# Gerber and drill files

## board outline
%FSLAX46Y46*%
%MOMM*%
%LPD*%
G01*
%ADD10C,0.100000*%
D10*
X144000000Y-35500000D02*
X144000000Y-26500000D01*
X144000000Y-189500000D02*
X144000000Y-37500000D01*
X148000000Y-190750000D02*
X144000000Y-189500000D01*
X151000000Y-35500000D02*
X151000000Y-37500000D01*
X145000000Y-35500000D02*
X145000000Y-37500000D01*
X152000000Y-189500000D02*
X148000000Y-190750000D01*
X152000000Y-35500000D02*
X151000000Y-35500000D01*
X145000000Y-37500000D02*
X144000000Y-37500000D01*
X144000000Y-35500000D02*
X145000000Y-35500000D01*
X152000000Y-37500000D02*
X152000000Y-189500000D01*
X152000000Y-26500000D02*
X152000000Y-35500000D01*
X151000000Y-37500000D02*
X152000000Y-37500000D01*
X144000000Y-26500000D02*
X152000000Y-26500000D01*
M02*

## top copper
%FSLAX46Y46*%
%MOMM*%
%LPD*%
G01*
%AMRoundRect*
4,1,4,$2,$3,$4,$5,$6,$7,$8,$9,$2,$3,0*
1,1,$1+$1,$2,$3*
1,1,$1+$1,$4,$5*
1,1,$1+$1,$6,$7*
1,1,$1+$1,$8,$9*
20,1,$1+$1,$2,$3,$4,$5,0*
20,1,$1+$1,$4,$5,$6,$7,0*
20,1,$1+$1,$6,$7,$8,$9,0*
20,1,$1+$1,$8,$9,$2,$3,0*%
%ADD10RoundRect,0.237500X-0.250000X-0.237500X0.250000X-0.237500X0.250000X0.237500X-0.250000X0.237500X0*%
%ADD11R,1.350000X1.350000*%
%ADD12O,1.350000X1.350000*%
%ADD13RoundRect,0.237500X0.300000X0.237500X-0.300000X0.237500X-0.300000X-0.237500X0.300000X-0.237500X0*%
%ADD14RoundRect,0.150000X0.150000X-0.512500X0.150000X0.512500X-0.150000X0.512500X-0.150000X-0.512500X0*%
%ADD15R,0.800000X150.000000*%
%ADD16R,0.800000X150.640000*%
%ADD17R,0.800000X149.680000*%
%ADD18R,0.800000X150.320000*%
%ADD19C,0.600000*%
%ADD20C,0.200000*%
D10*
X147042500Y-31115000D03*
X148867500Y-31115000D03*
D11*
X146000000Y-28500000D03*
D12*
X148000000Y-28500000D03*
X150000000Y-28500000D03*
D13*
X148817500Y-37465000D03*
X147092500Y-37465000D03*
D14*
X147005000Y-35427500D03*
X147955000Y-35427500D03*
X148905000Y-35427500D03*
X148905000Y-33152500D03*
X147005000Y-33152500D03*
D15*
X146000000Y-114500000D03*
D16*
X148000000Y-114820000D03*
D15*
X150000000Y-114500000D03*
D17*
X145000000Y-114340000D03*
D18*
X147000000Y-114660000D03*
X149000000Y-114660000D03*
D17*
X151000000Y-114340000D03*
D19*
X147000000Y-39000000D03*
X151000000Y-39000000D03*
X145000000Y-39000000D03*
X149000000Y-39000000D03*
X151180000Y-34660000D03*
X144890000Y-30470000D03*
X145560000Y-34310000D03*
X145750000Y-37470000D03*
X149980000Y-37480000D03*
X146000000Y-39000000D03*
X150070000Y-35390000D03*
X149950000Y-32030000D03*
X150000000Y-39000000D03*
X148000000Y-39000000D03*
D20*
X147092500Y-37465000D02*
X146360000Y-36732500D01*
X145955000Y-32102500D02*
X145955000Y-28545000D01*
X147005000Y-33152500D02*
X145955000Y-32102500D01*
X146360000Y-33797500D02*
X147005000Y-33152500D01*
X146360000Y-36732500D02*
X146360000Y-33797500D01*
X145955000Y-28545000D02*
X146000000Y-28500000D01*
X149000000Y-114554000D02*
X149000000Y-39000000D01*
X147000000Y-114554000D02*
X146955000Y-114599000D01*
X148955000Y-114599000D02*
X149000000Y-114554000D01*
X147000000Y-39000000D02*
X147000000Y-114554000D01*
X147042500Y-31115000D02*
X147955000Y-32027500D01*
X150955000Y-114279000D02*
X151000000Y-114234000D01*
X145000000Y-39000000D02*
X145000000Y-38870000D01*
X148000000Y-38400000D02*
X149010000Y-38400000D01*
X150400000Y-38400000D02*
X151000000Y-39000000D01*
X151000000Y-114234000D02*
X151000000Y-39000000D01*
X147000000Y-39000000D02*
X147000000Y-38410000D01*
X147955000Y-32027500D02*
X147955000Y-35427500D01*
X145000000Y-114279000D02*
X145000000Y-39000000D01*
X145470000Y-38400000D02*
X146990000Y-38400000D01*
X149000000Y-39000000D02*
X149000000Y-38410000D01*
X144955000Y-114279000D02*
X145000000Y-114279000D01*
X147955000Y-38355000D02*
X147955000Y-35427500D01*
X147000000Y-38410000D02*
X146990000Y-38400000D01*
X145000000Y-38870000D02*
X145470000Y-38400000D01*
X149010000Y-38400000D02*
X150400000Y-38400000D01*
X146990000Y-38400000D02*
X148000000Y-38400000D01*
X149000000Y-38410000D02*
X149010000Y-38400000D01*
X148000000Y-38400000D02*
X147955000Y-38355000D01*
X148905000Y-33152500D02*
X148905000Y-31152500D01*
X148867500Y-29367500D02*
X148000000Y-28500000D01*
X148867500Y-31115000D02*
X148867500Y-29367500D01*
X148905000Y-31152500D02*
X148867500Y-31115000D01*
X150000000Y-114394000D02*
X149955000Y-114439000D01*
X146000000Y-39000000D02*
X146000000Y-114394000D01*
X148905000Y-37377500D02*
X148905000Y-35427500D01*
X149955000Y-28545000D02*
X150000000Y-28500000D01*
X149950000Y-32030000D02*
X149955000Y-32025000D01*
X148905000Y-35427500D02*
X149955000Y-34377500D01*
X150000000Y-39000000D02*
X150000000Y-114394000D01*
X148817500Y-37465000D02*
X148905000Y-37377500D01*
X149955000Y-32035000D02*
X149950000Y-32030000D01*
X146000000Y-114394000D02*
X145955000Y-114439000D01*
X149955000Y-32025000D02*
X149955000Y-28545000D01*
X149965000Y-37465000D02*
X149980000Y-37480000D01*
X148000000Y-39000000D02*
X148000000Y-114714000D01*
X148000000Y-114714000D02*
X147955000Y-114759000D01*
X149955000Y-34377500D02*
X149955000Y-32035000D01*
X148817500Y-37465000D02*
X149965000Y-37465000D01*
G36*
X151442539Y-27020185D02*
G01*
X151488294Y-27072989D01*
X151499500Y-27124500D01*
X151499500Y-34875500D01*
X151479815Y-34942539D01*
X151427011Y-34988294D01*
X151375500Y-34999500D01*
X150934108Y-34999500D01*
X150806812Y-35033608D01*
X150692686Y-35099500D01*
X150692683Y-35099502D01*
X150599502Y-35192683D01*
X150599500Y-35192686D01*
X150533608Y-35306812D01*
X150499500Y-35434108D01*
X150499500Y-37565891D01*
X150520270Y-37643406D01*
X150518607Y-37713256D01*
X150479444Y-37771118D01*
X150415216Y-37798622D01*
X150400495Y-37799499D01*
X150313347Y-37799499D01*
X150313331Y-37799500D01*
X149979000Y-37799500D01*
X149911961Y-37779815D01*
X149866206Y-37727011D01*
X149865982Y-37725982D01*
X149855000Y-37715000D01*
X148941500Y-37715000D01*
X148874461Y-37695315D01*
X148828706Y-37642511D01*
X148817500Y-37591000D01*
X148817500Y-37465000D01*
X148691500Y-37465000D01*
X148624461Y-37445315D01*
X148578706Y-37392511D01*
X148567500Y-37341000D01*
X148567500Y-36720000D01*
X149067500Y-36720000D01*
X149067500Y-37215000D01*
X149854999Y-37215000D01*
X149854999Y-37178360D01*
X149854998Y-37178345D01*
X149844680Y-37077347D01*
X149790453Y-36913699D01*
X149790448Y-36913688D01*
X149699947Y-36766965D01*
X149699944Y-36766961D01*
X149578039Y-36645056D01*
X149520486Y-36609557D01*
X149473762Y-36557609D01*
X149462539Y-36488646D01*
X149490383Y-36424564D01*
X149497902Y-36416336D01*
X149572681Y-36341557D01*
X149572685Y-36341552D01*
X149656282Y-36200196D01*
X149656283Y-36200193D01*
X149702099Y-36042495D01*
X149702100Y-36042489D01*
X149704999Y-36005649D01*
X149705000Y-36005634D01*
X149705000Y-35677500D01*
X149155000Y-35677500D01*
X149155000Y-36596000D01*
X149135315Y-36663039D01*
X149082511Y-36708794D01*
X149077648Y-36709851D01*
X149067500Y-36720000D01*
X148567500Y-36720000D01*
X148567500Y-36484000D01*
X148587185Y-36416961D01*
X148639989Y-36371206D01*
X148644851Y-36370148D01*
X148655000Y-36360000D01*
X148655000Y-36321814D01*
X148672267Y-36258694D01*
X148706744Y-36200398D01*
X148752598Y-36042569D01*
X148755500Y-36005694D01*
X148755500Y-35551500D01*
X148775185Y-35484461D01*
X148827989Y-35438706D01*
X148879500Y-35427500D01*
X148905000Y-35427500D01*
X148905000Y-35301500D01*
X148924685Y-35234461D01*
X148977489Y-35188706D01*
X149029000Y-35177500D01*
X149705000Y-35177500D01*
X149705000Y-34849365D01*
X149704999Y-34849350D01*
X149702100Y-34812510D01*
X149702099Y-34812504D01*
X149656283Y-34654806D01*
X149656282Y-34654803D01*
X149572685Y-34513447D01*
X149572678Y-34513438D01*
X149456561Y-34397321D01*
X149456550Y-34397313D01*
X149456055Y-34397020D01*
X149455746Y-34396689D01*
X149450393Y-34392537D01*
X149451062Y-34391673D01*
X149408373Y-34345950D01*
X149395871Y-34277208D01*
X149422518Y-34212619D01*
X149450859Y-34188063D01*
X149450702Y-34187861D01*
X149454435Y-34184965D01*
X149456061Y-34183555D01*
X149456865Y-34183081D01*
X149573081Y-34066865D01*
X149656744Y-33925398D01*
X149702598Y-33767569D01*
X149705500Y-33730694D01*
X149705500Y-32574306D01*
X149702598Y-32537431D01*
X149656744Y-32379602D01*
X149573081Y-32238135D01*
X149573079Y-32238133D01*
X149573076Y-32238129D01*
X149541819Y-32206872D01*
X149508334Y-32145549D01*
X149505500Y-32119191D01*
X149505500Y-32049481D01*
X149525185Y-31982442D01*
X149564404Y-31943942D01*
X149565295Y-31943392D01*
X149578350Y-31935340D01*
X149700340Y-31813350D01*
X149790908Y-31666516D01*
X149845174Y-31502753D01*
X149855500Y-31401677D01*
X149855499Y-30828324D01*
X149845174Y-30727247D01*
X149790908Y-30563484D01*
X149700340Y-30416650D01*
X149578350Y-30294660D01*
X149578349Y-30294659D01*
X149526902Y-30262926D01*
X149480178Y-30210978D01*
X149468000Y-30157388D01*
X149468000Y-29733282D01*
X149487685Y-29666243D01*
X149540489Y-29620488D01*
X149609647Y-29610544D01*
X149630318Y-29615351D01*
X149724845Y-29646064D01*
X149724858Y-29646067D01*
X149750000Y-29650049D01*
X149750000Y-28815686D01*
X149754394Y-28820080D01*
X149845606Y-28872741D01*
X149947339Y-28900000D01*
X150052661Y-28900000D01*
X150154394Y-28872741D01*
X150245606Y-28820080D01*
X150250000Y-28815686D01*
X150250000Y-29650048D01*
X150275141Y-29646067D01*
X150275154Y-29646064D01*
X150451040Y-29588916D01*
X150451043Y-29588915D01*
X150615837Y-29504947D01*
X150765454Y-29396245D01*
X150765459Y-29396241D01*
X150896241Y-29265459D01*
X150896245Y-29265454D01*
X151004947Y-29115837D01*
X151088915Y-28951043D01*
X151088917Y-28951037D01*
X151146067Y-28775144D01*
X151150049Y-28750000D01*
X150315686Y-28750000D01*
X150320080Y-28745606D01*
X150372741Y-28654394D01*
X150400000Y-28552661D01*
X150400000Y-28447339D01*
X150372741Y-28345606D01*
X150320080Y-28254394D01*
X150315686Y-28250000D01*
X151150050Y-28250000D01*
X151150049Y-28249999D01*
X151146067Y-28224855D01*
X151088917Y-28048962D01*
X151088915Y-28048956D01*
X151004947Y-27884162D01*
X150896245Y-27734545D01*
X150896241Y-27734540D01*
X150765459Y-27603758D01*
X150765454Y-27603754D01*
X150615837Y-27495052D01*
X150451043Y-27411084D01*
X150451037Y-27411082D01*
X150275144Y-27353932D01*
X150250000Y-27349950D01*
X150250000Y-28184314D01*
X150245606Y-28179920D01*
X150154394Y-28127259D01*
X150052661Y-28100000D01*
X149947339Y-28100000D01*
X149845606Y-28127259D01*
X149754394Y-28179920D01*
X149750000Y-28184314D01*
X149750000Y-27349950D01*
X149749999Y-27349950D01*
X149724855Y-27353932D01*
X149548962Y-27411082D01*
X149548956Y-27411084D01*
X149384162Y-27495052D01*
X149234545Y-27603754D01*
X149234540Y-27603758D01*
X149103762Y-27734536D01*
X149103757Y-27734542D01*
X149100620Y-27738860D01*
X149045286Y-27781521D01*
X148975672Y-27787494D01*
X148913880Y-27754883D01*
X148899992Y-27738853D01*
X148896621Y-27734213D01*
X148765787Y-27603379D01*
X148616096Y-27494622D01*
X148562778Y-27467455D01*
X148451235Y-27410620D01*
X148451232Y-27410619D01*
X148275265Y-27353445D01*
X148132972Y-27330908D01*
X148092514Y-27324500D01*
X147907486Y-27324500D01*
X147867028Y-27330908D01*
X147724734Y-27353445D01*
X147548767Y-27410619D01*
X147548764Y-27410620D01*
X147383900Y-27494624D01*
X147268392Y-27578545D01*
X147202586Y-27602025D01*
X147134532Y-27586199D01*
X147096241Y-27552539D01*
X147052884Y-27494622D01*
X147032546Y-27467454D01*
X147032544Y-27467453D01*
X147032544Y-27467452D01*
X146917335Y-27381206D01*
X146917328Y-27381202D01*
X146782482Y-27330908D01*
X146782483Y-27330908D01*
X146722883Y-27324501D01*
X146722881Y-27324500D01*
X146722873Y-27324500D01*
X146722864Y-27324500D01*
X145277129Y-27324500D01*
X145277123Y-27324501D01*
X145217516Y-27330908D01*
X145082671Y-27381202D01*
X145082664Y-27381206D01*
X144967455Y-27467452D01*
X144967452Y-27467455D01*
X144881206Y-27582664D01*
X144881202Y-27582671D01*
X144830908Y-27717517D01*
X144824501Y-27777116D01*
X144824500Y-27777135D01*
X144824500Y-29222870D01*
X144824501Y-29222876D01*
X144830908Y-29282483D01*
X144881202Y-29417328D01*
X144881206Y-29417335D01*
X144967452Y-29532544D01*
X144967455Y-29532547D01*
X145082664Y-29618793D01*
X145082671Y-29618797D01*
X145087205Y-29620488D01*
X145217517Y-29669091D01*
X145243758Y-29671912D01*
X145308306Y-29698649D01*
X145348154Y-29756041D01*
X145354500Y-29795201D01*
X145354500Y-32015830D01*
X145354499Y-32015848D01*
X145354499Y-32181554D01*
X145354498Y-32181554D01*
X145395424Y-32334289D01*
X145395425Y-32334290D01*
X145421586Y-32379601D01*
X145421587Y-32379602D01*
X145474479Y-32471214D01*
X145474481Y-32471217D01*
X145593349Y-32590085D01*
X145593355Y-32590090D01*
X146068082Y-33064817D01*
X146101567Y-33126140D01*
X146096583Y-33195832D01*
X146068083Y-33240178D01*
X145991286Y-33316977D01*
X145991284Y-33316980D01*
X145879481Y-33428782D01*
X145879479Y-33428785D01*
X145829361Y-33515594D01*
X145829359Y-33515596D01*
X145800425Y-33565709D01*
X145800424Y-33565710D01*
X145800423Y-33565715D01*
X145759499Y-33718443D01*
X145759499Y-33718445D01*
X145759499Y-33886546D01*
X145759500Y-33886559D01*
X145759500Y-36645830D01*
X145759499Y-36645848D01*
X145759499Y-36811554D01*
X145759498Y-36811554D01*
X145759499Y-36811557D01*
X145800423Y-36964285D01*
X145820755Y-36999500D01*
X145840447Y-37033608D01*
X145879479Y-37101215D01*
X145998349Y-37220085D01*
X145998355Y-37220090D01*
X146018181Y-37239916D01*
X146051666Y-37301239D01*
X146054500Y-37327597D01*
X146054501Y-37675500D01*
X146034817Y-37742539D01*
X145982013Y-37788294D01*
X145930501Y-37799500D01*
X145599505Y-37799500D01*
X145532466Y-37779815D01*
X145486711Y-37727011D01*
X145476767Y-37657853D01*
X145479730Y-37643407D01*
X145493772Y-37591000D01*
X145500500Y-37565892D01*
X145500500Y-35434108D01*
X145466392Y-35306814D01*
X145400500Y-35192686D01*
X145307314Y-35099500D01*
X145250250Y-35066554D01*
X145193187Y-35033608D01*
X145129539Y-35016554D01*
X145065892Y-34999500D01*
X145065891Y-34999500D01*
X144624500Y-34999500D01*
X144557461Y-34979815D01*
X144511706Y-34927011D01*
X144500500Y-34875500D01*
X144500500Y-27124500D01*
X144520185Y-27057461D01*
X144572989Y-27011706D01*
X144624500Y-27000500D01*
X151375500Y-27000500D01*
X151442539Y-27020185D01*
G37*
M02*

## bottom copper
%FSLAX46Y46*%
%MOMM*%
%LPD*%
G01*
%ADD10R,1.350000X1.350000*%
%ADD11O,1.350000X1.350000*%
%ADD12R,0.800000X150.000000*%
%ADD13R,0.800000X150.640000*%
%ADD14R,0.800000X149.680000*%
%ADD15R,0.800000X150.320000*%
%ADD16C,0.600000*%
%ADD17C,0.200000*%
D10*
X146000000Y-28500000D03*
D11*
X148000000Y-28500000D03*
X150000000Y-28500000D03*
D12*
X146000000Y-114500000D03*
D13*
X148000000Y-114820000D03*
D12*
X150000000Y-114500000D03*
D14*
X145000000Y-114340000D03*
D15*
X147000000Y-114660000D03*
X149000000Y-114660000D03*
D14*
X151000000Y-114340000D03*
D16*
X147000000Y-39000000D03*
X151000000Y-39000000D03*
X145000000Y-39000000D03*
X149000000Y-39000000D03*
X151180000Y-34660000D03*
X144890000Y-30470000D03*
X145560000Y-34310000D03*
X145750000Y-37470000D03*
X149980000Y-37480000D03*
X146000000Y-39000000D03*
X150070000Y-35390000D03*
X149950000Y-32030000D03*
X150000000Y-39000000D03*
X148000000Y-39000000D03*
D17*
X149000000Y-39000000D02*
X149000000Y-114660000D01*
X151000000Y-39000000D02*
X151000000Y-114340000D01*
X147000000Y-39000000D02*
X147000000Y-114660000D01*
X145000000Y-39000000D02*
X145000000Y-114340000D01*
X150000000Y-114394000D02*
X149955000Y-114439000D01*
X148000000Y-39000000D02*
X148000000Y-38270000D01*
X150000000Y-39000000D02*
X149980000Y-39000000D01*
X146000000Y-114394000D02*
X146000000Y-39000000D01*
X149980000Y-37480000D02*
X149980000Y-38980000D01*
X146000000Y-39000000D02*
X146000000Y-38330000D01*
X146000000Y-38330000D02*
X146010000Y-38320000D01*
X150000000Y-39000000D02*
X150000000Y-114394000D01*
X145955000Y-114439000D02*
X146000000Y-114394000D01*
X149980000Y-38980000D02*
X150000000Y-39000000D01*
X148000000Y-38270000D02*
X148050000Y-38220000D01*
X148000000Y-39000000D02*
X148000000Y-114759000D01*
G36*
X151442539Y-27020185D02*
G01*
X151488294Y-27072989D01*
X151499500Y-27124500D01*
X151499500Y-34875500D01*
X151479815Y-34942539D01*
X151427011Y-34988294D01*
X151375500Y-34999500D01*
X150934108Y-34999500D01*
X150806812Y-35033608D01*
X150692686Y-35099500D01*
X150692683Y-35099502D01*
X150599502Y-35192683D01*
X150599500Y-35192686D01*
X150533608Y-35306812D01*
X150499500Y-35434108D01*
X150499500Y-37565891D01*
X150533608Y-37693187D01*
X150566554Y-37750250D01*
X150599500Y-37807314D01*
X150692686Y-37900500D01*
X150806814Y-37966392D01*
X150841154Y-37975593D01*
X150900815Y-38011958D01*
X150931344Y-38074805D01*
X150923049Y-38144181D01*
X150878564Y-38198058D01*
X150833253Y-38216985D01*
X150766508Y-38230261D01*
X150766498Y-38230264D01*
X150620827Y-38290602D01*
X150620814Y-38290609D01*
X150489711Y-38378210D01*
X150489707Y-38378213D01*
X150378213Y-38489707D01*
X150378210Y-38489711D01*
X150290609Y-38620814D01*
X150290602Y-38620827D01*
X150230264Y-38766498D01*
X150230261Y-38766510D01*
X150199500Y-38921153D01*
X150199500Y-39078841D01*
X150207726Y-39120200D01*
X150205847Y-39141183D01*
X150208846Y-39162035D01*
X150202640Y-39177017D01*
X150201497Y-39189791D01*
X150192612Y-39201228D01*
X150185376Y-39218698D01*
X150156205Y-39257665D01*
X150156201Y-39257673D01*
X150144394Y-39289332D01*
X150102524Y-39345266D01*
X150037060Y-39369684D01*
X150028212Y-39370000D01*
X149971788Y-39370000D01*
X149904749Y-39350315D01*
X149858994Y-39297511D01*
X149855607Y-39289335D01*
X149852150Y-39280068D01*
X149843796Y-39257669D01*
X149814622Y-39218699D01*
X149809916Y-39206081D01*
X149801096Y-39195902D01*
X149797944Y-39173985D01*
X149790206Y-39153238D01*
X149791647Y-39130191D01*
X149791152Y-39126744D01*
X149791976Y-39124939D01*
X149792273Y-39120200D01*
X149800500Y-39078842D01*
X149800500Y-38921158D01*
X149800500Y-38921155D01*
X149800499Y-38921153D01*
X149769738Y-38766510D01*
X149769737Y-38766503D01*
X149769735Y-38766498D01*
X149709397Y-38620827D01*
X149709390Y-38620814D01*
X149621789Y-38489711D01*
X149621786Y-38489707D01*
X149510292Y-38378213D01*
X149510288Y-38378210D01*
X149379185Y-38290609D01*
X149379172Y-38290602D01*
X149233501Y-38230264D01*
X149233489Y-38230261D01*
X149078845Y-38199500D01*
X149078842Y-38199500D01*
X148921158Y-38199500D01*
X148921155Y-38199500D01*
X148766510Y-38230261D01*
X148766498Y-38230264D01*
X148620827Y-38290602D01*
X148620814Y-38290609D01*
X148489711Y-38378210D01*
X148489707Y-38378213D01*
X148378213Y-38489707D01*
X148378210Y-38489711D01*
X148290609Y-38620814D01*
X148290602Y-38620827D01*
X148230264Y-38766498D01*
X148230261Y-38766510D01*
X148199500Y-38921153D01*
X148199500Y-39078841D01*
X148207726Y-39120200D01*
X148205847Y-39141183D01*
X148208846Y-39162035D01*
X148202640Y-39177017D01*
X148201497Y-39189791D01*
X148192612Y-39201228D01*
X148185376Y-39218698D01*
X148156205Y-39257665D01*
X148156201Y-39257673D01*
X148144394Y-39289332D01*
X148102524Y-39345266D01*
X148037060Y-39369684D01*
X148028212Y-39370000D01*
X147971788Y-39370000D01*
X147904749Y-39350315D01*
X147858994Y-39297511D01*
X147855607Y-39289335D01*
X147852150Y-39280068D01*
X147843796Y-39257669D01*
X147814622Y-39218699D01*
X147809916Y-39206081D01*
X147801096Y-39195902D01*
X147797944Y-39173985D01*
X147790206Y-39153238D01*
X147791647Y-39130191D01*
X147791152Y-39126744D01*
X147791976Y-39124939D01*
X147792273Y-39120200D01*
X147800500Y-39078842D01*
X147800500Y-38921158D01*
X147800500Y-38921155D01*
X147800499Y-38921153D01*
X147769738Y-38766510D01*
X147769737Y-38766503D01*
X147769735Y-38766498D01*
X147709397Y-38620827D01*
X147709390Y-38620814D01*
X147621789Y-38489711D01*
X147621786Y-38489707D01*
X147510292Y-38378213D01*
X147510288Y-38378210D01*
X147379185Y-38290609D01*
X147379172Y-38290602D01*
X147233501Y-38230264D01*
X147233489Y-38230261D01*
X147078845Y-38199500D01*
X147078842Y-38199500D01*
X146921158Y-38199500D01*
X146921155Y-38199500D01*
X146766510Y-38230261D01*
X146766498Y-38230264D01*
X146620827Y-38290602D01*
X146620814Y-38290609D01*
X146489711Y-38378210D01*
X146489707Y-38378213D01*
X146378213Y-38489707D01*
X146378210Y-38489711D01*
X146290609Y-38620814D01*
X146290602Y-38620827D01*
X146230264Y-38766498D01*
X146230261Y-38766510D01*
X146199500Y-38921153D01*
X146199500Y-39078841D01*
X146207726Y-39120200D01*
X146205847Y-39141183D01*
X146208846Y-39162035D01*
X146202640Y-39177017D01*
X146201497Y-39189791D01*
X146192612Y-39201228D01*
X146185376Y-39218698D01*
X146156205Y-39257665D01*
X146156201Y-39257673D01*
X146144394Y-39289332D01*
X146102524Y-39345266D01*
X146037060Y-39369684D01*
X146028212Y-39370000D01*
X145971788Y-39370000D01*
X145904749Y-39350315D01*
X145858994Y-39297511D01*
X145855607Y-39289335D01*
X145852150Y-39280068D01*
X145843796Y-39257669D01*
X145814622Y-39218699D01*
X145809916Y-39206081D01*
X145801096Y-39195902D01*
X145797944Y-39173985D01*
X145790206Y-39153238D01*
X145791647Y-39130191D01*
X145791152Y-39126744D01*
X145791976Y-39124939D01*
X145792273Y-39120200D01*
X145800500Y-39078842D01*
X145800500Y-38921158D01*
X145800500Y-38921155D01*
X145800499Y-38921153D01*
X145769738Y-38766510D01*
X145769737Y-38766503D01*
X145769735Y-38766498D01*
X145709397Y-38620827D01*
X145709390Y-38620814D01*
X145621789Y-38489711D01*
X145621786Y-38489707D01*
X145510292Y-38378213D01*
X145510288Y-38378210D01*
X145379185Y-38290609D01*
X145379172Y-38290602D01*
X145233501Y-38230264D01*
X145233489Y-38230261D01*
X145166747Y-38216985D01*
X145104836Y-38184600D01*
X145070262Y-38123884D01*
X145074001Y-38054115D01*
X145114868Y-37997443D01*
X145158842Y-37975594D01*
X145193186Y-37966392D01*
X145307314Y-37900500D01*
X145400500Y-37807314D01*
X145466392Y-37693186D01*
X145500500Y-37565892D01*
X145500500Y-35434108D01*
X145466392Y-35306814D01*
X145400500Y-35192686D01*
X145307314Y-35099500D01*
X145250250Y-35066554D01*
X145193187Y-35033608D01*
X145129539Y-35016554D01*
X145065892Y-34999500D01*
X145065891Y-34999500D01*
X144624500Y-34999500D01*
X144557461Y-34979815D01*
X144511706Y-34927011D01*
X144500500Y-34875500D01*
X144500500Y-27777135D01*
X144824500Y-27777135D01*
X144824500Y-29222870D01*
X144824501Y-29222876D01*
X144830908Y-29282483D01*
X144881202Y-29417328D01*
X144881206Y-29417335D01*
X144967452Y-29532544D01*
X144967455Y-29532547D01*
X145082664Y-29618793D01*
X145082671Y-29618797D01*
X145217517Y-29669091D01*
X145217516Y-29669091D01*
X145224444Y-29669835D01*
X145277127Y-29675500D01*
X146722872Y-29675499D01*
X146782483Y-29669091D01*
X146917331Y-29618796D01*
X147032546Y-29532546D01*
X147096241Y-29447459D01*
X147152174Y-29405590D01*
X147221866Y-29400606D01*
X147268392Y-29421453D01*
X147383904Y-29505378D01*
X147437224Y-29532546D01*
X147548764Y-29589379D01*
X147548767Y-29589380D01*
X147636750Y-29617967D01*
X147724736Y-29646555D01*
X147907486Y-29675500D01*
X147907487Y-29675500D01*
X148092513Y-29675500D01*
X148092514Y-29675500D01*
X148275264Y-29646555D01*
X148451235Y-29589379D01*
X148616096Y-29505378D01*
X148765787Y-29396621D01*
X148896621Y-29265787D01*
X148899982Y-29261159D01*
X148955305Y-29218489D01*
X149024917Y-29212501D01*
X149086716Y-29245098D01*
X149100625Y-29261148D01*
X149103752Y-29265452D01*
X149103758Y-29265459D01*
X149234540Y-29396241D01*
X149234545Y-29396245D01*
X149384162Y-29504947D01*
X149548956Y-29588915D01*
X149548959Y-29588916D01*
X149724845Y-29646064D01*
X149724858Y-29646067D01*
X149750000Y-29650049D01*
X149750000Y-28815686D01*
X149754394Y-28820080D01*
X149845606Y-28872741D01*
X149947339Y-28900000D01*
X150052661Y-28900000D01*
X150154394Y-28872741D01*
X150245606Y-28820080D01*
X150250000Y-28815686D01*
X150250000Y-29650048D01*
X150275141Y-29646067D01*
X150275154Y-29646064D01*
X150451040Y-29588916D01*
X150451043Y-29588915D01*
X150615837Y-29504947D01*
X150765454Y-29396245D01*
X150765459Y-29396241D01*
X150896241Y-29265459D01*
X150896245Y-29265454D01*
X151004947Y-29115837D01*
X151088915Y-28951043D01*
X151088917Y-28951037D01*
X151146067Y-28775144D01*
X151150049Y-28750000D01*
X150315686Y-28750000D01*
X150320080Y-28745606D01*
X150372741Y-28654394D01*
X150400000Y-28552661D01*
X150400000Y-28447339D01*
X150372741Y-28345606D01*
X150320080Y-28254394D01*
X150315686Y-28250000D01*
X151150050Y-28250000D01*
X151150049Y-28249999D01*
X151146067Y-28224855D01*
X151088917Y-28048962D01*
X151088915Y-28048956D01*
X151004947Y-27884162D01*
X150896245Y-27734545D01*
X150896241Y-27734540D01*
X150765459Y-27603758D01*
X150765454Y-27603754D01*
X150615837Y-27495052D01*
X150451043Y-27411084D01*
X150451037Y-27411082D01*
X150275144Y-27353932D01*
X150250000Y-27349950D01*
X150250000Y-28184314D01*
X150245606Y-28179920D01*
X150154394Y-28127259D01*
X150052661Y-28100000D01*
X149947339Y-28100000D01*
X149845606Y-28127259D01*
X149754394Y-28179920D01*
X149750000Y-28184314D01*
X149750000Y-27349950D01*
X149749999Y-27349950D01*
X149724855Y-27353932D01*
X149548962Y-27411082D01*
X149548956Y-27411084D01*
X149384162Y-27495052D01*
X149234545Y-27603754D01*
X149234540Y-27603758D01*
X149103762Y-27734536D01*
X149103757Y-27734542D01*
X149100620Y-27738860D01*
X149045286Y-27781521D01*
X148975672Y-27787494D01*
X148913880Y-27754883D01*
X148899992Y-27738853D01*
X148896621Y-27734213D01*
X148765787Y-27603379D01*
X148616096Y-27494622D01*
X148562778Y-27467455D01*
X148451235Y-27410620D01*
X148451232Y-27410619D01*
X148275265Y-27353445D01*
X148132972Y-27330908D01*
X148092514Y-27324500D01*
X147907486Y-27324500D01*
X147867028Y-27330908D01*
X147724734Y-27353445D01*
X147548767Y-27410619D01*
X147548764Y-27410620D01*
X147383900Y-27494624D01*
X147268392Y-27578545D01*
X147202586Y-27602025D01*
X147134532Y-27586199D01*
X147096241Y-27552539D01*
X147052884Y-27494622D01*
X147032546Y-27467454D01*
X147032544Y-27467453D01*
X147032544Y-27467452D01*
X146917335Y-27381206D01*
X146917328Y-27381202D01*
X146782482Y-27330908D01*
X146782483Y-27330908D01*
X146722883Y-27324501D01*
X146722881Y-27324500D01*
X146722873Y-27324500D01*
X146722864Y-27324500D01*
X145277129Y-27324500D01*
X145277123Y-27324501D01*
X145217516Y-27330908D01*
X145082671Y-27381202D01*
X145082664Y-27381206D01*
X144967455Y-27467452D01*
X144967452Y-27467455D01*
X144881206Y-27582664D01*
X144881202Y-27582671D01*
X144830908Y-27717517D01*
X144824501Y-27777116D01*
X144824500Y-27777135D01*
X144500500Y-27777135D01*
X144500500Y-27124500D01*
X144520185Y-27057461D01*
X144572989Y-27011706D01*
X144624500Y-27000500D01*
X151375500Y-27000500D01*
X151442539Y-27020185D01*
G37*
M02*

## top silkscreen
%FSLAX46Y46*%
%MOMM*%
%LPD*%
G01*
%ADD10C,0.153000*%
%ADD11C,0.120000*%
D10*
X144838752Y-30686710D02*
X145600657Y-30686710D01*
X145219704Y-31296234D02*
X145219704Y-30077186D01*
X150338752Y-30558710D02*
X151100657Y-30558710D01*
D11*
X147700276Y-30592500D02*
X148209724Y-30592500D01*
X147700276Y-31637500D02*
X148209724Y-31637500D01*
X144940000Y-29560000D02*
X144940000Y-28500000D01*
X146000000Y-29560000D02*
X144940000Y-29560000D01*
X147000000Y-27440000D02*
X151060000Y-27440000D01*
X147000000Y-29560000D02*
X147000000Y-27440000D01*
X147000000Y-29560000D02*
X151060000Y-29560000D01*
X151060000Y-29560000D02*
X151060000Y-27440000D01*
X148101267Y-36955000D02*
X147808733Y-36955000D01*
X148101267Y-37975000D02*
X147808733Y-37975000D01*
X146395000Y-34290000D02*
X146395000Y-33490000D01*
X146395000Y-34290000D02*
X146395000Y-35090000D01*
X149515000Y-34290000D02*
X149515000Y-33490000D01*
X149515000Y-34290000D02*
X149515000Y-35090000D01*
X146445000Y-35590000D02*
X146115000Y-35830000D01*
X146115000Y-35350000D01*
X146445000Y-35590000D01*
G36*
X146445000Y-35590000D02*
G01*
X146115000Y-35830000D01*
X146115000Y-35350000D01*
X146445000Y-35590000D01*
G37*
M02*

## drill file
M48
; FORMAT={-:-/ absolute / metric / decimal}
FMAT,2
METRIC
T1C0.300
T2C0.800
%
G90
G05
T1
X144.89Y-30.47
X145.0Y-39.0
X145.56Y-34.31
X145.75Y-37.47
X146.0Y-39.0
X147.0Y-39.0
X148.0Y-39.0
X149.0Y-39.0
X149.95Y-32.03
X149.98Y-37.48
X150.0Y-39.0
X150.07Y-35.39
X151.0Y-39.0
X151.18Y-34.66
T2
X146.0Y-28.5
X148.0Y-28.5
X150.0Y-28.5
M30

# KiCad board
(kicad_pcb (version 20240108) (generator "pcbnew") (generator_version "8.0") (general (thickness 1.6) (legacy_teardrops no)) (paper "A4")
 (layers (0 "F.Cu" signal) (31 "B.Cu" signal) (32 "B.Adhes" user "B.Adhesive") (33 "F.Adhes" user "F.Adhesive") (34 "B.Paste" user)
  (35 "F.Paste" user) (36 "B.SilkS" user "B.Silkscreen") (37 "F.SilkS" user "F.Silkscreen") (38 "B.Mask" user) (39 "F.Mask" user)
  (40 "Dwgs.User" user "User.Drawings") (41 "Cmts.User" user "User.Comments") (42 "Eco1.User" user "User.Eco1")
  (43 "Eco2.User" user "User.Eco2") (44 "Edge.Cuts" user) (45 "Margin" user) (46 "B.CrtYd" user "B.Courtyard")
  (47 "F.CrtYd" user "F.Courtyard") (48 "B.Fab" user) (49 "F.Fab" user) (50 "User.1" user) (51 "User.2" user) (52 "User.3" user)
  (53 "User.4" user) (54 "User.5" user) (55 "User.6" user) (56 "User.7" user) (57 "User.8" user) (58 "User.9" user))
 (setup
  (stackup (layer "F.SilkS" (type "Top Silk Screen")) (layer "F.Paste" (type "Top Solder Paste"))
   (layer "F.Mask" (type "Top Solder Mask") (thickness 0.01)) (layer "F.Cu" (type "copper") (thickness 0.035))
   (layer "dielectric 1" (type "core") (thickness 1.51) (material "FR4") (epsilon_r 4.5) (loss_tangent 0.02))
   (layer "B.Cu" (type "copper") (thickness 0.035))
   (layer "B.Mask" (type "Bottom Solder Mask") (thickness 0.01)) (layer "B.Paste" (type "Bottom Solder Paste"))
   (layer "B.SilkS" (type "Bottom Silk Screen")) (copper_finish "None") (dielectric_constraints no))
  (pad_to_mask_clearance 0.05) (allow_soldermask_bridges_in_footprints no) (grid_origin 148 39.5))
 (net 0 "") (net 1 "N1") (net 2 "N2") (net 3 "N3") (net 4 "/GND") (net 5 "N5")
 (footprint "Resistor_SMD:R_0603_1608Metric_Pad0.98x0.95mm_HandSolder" (layer "F.Cu") (at 147.955 31.115)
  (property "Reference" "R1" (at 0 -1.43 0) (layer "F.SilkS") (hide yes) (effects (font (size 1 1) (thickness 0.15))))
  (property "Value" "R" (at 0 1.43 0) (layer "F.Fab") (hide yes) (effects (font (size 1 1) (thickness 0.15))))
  (fp_line (start -0.254724 -0.5225) (end 0.254724 -0.5225) (stroke (width 0.12) (type solid)) (layer "F.SilkS"))
  (fp_line (start -0.254724 0.5225) (end 0.254724 0.5225) (stroke (width 0.12) (type solid)) (layer "F.SilkS"))
  (pad "1" smd roundrect (at -0.9125 0) (size 0.975 0.95) (layers "F.Cu" "F.Paste" "F.Mask") (roundrect_rratio 0.25) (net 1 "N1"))
  (pad "2" smd roundrect (at 0.9125 0) (size 0.975 0.95) (layers "F.Cu" "F.Paste" "F.Mask") (roundrect_rratio 0.25) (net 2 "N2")))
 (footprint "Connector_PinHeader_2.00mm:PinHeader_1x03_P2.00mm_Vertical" (layer "F.Cu") (at 146 28.5 90)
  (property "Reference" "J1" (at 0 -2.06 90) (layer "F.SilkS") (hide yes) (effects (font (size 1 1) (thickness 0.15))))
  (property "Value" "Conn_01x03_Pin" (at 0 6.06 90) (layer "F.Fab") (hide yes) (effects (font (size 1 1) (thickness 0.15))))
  (fp_line (start -1.06 -1.06) (end 0 -1.06) (stroke (width 0.12) (type solid)) (layer "F.SilkS"))
  (fp_line (start -1.06 0) (end -1.06 -1.06) (stroke (width 0.12) (type solid)) (layer "F.SilkS"))
  (fp_line (start 1.06 1) (end 1.06 5.06) (stroke (width 0.12) (type solid)) (layer "F.SilkS"))
  (fp_line (start -1.06 1) (end 1.06 1) (stroke (width 0.12) (type solid)) (layer "F.SilkS"))
  (fp_line (start -1.06 1) (end -1.06 5.06) (stroke (width 0.12) (type solid)) (layer "F.SilkS"))
  (fp_line (start -1.06 5.06) (end 1.06 5.06) (stroke (width 0.12) (type solid)) (layer "F.SilkS"))
  (pad "1" thru_hole rect (at 0 0 90) (size 1.35 1.35) (drill 0.8) (layers "*.Cu" "*.Mask") (remove_unused_layers no) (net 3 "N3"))
  (pad "2" thru_hole oval (at 0 2 90) (size 1.35 1.35) (drill 0.8) (layers "*.Cu" "*.Mask") (remove_unused_layers no) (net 2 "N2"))
  (pad "3" thru_hole oval (at 0 4 90) (size 1.35 1.35) (drill 0.8) (layers "*.Cu" "*.Mask") (remove_unused_layers no) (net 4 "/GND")))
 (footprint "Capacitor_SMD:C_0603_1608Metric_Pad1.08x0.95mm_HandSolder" (layer "F.Cu") (at 147.955 37.465 180)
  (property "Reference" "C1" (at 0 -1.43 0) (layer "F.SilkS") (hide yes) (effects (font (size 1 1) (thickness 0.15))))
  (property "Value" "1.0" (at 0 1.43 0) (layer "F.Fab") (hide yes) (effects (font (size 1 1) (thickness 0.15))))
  (fp_line (start -0.146267 0.51) (end 0.146267 0.51) (stroke (width 0.12) (type solid)) (layer "F.SilkS"))
  (fp_line (start -0.146267 -0.51) (end 0.146267 -0.51) (stroke (width 0.12) (type solid)) (layer "F.SilkS"))
  (pad "1" smd roundrect (at -0.8625 0 180) (size 1.075 0.95) (layers "F.Cu" "F.Paste" "F.Mask") (roundrect_rratio 0.25) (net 4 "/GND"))
  (pad "2" smd roundrect (at 0.8625 0 180) (size 1.075 0.95) (layers "F.Cu" "F.Paste" "F.Mask") (roundrect_rratio 0.25) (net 3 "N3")))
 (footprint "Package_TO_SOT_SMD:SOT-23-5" (layer "F.Cu") (at 147.955 34.29 90)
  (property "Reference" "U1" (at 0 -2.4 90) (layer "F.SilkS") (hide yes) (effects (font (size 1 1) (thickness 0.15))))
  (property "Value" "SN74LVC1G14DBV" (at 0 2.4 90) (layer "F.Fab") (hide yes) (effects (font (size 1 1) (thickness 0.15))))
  (fp_line (start 0 -1.56) (end 0.8 -1.56) (stroke (width 0.12) (type solid)) (layer "F.SilkS"))
  (fp_line (start 0 -1.56) (end -0.8 -1.56) (stroke (width 0.12) (type solid)) (layer "F.SilkS"))
  (fp_line (start 0 1.56) (end 0.8 1.56) (stroke (width 0.12) (type solid)) (layer "F.SilkS"))
  (fp_line (start 0 1.56) (end -0.8 1.56) (stroke (width 0.12) (type solid)) (layer "F.SilkS"))
  (fp_poly
   (pts (xy -1.3 -1.51) (xy -1.54 -1.84) (xy -1.06 -1.84) (xy -1.3 -1.51)) (stroke (width 0.12) (type solid)) (fill solid) (layer "F.SilkS"))
  (pad "1" smd roundrect (at -1.1375 -0.95 90) (size 1.325 0.6) (layers "F.Cu" "F.Paste" "F.Mask") (roundrect_rratio 0.25) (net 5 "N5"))
  (pad "2" smd roundrect (at -1.1375 0 90) (size 1.325 0.6) (layers "F.Cu" "F.Paste" "F.Mask") (roundrect_rratio 0.25) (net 1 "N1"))
  (pad "3" smd roundrect (at -1.1375 0.95 90) (size 1.325 0.6) (layers "F.Cu" "F.Paste" "F.Mask") (roundrect_rratio 0.25) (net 4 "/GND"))
  (pad "4" smd roundrect (at 1.1375 0.95 90) (size 1.325 0.6) (layers "F.Cu" "F.Paste" "F.Mask") (roundrect_rratio 0.25) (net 2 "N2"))
  (pad "5" smd roundrect (at 1.1375 -0.95 90) (size 1.325 0.6) (layers "F.Cu" "F.Paste" "F.Mask") (roundrect_rratio 0.25) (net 3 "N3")))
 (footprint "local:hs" (layer "F.Cu") (at 148 39.5)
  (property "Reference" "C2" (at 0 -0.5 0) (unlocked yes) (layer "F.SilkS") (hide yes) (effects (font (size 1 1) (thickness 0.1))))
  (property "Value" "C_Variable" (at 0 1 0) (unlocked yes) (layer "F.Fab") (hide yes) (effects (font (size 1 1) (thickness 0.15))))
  (pad "1" smd rect (at -2 75) (size 0.8 150) (layers "F.Cu") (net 4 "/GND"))
  (pad "1" smd rect (at -2 75) (size 0.8 150) (layers "B.Cu") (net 4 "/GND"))
  (pad "1" smd rect (at 0 75.32) (size 0.8 150.64) (layers "F.Cu") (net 4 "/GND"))
  (pad "1" smd rect (at 0 75.32) (size 0.8 150.64) (layers "B.Cu") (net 4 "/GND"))
  (pad "1" smd rect (at 2 75) (size 0.8 150) (layers "F.Cu") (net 4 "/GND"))
  (pad "1" smd rect (at 2 75) (size 0.8 150) (layers "B.Cu") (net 4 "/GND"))
  (pad "2" smd rect (at -3 74.84) (size 0.8 149.68) (layers "F.Cu") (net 1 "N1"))
  (pad "2" smd rect (at -3 74.84) (size 0.8 149.68) (layers "B.Cu") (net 1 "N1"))
  (pad "2" smd rect (at -1 75.16) (size 0.8 150.32) (layers "F.Cu") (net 1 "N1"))
  (pad "2" smd rect (at -1 75.16) (size 0.8 150.32) (layers "B.Cu") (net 1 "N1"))
  (pad "2" smd rect (at 1 75.16) (size 0.8 150.32) (layers "F.Cu") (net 1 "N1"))
  (pad "2" smd rect (at 1 75.16) (size 0.8 150.32) (layers "B.Cu") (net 1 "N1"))
  (pad "2" smd rect (at 3 74.84) (size 0.8 149.68) (layers "F.Cu") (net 1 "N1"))
  (pad "2" smd rect (at 3 74.84) (size 0.8 149.68) (layers "B.Cu") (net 1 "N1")))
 (gr_line (start 144 35.5) (end 144 26.5) (stroke (width 0.1) (type default)) (layer "Edge.Cuts"))
 (gr_line (start 144 189.5) (end 144 37.5) (stroke (width 0.1) (type default)) (layer "Edge.Cuts"))
 (gr_line (start 148 190.75) (end 144 189.5) (stroke (width 0.1) (type default)) (layer "Edge.Cuts"))
 (gr_line (start 151 35.5) (end 151 37.5) (stroke (width 0.1) (type default)) (layer "Edge.Cuts"))
 (gr_line (start 145 35.5) (end 145 37.5) (stroke (width 0.1) (type default)) (layer "Edge.Cuts"))
 (gr_line (start 152 189.5) (end 148 190.75) (stroke (width 0.1) (type default)) (layer "Edge.Cuts"))
 (gr_line (start 152 35.5) (end 151 35.5) (stroke (width 0.1) (type default)) (layer "Edge.Cuts"))
 (gr_line (start 145 37.5) (end 144 37.5) (stroke (width 0.1) (type default)) (layer "Edge.Cuts"))
 (gr_line (start 144 35.5) (end 145 35.5) (stroke (width 0.1) (type default)) (layer "Edge.Cuts"))
 (gr_line (start 152 37.5) (end 152 189.5) (stroke (width 0.1) (type default)) (layer "Edge.Cuts"))
 (gr_line (start 152 26.5) (end 152 35.5) (stroke (width 0.1) (type default)) (layer "Edge.Cuts"))
 (gr_line (start 151 37.5) (end 152 37.5) (stroke (width 0.1) (type default)) (layer "Edge.Cuts"))
 (gr_line (start 144 26.5) (end 152 26.5) (stroke (width 0.1) (type default)) (layer "Edge.Cuts"))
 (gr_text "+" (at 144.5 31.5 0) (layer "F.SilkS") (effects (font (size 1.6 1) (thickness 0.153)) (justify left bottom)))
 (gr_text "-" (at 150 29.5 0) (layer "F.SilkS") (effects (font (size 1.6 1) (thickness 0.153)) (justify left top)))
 (segment (start 147.0925 37.465) (end 146.36 36.7325) (width 0.2) (layer "F.Cu") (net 3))
 (segment (start 145.955 32.1025) (end 145.955 28.545) (width 0.2) (layer "F.Cu") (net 3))
 (segment (start 147.005 33.1525) (end 145.955 32.1025) (width 0.2) (layer "F.Cu") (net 3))
 (segment (start 146.36 33.7975) (end 147.005 33.1525) (width 0.2) (layer "F.Cu") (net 3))
 (segment (start 146.36 36.7325) (end 146.36 33.7975) (width 0.2) (layer "F.Cu") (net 3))
 (segment (start 145.955 28.545) (end 146 28.5) (width 0.2) (layer "F.Cu") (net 3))
 (segment (start 149 114.554) (end 149 39) (width 0.2) (layer "F.Cu") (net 1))
 (segment (start 147 114.554) (end 146.955 114.599) (width 0.2) (layer "F.Cu") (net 1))
 (segment (start 148.955 114.599) (end 149 114.554) (width 0.2) (layer "F.Cu") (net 1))
 (segment (start 147 39) (end 147 114.554) (width 0.2) (layer "F.Cu") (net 1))
 (segment (start 147.0425 31.115) (end 147.955 32.0275) (width 0.2) (layer "F.Cu") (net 1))
 (segment (start 150.955 114.279) (end 151 114.234) (width 0.2) (layer "F.Cu") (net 1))
 (segment (start 145 39) (end 145 38.87) (width 0.2) (layer "F.Cu") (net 1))
 (segment (start 148 38.4) (end 149.01 38.4) (width 0.2) (layer "F.Cu") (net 1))
 (segment (start 150.4 38.4) (end 151 39) (width 0.2) (layer "F.Cu") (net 1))
 (segment (start 151 114.234) (end 151 39) (width 0.2) (layer "F.Cu") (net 1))
 (segment (start 147 39) (end 147 38.41) (width 0.2) (layer "F.Cu") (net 1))
 (segment (start 147.955 32.0275) (end 147.955 35.4275) (width 0.2) (layer "F.Cu") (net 1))
 (segment (start 145 114.279) (end 145 39) (width 0.2) (layer "F.Cu") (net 1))
 (segment (start 145.47 38.4) (end 146.99 38.4) (width 0.2) (layer "F.Cu") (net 1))
 (segment (start 149 39) (end 149 38.41) (width 0.2) (layer "F.Cu") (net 1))
 (segment (start 144.955 114.279) (end 145 114.279) (width 0.2) (layer "F.Cu") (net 1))
 (segment (start 147.955 38.355) (end 147.955 35.4275) (width 0.2) (layer "F.Cu") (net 1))
 (segment (start 147 38.41) (end 146.99 38.4) (width 0.2) (layer "F.Cu") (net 1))
 (segment (start 145 38.87) (end 145.47 38.4) (width 0.2) (layer "F.Cu") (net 1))
 (segment (start 149.01 38.4) (end 150.4 38.4) (width 0.2) (layer "F.Cu") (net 1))
 (segment (start 146.99 38.4) (end 148 38.4) (width 0.2) (layer "F.Cu") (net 1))
 (segment (start 149 38.41) (end 149.01 38.4) (width 0.2) (layer "F.Cu") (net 1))
 (segment (start 148 38.4) (end 147.955 38.355) (width 0.2) (layer "F.Cu") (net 1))
 (via (at 147 39) (size 0.6) (drill 0.3) (layers "F.Cu" "B.Cu") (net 1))
 (via (at 151 39) (size 0.6) (drill 0.3) (layers "F.Cu" "B.Cu") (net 1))
 (via (at 145 39) (size 0.6) (drill 0.3) (layers "F.Cu" "B.Cu") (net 1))
 (via (at 149 39) (size 0.6) (drill 0.3) (layers "F.Cu" "B.Cu") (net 1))
 (segment (start 149 39) (end 149 114.66) (width 0.2) (layer "B.Cu") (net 1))
 (segment (start 151 39) (end 151 114.34) (width 0.2) (layer "B.Cu") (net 1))
 (segment (start 147 39) (end 147 114.66) (width 0.2) (layer "B.Cu") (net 1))
 (segment (start 145 39) (end 145 114.34) (width 0.2) (layer "B.Cu") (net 1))
 (segment (start 148.905 33.1525) (end 148.905 31.1525) (width 0.2) (layer "F.Cu") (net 2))
 (segment (start 148.8675 29.3675) (end 148 28.5) (width 0.2) (layer "F.Cu") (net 2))
 (segment (start 148.8675 31.115) (end 148.8675 29.3675) (width 0.2) (layer "F.Cu") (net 2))
 (segment (start 148.905 31.1525) (end 148.8675 31.115) (width 0.2) (layer "F.Cu") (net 2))
 (segment (start 150 114.394) (end 149.955 114.439) (width 0.2) (layer "F.Cu") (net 4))
 (segment (start 146 39) (end 146 114.394) (width 0.2) (layer "F.Cu") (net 4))
 (segment (start 148.905 37.3775) (end 148.905 35.4275) (width 0.2) (layer "F.Cu") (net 4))
 (segment (start 149.955 28.545) (end 150 28.5) (width 0.2) (layer "F.Cu") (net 4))
 (segment (start 149.95 32.03) (end 149.955 32.025) (width 0.2) (layer "F.Cu") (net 4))
 (segment (start 148.905 35.4275) (end 149.955 34.3775) (width 0.2) (layer "F.Cu") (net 4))
 (segment (start 150 39) (end 150 114.394) (width 0.2) (layer "F.Cu") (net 4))
 (segment (start 148.8175 37.465) (end 148.905 37.3775) (width 0.2) (layer "F.Cu") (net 4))
 (segment (start 149.955 32.035) (end 149.95 32.03) (width 0.2) (layer "F.Cu") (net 4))
 (segment (start 146 114.394) (end 145.955 114.439) (width 0.2) (layer "F.Cu") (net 4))
 (segment (start 149.955 32.025) (end 149.955 28.545) (width 0.2) (layer "F.Cu") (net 4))
 (segment (start 149.965 37.465) (end 149.98 37.48) (width 0.2) (layer "F.Cu") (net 4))
 (segment (start 148 39) (end 148 114.714) (width 0.2) (layer "F.Cu") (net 4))
 (segment (start 148 114.714) (end 147.955 114.759) (width 0.2) (layer "F.Cu") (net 4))
 (segment (start 149.955 34.3775) (end 149.955 32.035) (width 0.2) (layer "F.Cu") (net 4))
 (segment (start 148.8175 37.465) (end 149.965 37.465) (width 0.2) (layer "F.Cu") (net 4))
 (via (at 151.18 34.66) (size 0.6) (drill 0.3) (layers "F.Cu" "B.Cu") (free yes) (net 4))
 (via (at 144.89 30.47) (size 0.6) (drill 0.3) (layers "F.Cu" "B.Cu") (free yes) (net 4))
 (via (at 145.56 34.31) (size 0.6) (drill 0.3) (layers "F.Cu" "B.Cu") (free yes) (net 4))
 (via (at 145.75 37.47) (size 0.6) (drill 0.3) (layers "F.Cu" "B.Cu") (free yes) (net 4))
 (via (at 149.98 37.48) (size 0.6) (drill 0.3) (layers "F.Cu" "B.Cu") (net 4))
 (via (at 146 39) (size 0.6) (drill 0.3) (layers "F.Cu" "B.Cu") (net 4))
 (via (at 150.07 35.39) (size 0.6) (drill 0.3) (layers "F.Cu" "B.Cu") (free yes) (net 4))
 (via (at 149.95 32.03) (size 0.6) (drill 0.3) (layers "F.Cu" "B.Cu") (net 4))
 (via (at 150 39) (size 0.6) (drill 0.3) (layers "F.Cu" "B.Cu") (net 4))
 (via (at 148 39) (size 0.6) (drill 0.3) (layers "F.Cu" "B.Cu") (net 4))
 (segment (start 150 114.394) (end 149.955 114.439) (width 0.2) (layer "B.Cu") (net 4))
 (segment (start 148 39) (end 148 38.27) (width 0.2) (layer "B.Cu") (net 4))
 (segment (start 150 39) (end 149.98 39) (width 0.2) (layer "B.Cu") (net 4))
 (segment (start 146 114.394) (end 146 39) (width 0.2) (layer "B.Cu") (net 4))
 (segment (start 149.98 37.48) (end 149.98 38.98) (width 0.2) (layer "B.Cu") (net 4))
 (segment (start 146 39) (end 146 38.33) (width 0.2) (layer "B.Cu") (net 4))
 (segment (start 146 38.33) (end 146.01 38.32) (width 0.2) (layer "B.Cu") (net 4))
 (segment (start 150 39) (end 150 114.394) (width 0.2) (layer "B.Cu") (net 4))
 (segment (start 145.955 114.439) (end 146 114.394) (width 0.2) (layer "B.Cu") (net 4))
 (segment (start 149.98 38.98) (end 150 39) (width 0.2) (layer "B.Cu") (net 4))
 (segment (start 148 38.27) (end 148.05 38.22) (width 0.2) (layer "B.Cu") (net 4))
 (segment (start 148 39) (end 148 114.759) (width 0.2) (layer "B.Cu") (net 4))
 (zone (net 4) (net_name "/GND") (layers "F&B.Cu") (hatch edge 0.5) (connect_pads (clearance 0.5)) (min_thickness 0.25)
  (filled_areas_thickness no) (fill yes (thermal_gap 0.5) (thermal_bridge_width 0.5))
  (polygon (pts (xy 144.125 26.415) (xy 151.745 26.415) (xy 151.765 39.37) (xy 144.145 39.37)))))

